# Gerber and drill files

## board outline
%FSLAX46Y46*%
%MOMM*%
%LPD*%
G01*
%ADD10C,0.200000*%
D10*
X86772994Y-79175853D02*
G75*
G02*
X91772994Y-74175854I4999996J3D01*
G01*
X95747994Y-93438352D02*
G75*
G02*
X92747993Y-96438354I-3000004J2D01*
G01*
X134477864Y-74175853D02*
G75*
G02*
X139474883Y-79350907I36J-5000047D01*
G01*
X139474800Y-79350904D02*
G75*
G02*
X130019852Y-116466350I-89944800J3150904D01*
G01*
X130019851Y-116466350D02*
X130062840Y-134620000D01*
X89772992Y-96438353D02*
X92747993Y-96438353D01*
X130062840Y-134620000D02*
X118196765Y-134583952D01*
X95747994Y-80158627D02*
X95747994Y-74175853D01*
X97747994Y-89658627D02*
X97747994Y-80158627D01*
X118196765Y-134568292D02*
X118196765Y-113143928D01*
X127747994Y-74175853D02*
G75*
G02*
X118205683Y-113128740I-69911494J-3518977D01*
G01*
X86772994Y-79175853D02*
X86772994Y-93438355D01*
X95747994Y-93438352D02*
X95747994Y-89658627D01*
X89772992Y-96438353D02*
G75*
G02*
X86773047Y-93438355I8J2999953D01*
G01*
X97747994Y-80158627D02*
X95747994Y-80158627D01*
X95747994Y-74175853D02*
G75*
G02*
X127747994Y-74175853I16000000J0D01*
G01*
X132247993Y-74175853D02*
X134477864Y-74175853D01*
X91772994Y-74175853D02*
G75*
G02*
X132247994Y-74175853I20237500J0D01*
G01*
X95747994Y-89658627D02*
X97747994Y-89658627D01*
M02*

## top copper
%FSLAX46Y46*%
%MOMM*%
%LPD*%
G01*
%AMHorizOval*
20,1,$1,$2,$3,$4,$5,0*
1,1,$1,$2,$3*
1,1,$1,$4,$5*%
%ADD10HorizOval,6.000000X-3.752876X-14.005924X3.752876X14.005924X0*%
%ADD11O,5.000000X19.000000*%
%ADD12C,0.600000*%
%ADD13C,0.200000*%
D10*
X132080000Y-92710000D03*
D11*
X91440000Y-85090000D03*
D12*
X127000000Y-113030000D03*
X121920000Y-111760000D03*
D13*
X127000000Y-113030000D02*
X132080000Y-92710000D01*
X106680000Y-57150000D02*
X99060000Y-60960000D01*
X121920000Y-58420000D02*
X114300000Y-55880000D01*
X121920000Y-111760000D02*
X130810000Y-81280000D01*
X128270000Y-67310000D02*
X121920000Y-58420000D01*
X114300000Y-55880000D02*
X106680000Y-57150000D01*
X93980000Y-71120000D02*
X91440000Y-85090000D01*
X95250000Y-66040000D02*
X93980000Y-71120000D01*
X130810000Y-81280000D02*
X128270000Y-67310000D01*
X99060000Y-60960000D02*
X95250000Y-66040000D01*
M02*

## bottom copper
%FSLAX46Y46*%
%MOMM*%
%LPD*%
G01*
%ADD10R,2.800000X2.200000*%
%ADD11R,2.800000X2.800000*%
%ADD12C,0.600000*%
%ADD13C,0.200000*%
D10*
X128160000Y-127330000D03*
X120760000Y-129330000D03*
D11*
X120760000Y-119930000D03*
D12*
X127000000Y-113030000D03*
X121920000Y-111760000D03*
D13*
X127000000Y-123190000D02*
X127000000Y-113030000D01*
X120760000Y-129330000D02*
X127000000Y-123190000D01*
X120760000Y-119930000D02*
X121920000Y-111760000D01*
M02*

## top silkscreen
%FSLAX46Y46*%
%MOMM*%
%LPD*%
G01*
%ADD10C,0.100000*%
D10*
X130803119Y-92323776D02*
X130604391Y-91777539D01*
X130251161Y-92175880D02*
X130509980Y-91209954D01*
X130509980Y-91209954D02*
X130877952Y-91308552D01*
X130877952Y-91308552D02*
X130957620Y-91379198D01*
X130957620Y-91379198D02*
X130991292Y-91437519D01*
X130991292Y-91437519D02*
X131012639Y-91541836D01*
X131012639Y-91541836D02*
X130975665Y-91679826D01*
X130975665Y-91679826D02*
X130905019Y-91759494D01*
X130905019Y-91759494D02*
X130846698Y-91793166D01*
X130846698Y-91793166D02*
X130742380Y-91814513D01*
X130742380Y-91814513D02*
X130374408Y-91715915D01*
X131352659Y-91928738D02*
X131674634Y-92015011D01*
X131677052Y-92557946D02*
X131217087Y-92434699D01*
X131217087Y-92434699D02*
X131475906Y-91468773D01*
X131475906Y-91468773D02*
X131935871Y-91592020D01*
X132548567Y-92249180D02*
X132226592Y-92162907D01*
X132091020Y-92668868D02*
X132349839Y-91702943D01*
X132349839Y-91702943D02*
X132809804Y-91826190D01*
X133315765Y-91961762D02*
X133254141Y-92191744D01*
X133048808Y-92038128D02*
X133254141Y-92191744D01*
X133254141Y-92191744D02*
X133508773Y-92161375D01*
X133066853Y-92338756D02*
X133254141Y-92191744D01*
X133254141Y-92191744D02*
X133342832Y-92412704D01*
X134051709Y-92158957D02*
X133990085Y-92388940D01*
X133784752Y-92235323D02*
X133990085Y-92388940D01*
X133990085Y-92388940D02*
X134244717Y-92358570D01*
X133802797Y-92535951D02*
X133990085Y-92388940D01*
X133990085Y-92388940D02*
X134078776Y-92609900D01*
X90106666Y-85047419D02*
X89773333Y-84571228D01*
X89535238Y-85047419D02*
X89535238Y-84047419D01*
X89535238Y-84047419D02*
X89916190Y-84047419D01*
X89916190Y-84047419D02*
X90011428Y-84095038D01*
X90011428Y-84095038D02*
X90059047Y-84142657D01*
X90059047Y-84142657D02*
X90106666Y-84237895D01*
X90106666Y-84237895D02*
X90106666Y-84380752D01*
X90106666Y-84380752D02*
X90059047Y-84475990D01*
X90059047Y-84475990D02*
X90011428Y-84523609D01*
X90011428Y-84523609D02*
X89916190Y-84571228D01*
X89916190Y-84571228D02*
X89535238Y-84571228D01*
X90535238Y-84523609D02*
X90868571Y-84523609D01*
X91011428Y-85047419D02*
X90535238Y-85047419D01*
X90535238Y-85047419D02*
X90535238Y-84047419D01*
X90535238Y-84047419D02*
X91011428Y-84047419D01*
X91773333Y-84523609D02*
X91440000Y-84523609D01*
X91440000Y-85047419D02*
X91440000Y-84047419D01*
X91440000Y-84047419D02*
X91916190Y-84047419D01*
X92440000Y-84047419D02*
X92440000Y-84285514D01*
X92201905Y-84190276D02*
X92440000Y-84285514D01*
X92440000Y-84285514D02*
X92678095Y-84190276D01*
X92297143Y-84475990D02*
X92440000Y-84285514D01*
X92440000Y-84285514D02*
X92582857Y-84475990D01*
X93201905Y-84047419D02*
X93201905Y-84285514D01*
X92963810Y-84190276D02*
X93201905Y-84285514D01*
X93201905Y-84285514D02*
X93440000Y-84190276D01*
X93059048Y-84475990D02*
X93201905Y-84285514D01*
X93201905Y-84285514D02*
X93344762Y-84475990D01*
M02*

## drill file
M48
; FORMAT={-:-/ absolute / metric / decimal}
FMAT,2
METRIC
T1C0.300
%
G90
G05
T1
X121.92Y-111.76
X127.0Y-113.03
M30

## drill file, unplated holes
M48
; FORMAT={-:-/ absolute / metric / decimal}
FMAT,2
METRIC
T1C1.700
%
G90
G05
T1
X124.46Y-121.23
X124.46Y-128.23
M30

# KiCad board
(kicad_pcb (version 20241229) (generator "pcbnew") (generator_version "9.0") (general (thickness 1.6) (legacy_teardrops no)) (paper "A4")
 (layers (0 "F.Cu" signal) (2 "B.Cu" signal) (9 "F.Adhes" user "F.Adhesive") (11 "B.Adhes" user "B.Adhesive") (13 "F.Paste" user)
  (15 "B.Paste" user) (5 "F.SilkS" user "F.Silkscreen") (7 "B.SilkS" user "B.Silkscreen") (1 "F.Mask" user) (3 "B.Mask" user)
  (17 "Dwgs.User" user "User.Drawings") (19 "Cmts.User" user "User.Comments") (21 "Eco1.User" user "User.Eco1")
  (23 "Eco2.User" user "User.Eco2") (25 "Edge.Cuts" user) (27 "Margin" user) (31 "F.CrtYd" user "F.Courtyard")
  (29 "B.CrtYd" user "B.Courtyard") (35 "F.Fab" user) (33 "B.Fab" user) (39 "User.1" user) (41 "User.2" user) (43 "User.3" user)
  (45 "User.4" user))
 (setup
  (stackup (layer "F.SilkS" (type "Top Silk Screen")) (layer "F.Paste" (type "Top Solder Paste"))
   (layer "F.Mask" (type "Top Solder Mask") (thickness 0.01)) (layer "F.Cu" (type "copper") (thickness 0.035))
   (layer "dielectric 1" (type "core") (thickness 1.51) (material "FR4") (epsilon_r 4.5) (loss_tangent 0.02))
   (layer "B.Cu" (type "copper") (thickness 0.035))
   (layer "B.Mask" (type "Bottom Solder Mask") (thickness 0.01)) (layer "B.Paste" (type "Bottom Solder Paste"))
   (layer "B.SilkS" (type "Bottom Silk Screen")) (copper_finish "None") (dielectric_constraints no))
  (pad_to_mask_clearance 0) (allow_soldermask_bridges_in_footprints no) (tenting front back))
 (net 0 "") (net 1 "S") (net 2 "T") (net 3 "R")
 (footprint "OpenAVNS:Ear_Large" (layer "F.Cu") (at 132.08 92.71 -15)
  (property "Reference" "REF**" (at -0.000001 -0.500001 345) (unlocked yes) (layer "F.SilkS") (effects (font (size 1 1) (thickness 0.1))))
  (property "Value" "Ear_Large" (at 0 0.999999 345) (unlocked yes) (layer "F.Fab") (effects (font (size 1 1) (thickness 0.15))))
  (pad "1" smd oval (at 0 0 345) (size 6 35) (layers "F.Cu" "F.Mask" "F.Paste") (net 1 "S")))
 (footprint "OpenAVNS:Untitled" (layer "F.Cu") (at 91.44 85.09)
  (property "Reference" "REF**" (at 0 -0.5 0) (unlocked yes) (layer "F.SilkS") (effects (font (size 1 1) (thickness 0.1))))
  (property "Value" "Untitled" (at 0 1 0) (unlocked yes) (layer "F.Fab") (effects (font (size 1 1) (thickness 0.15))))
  (pad "1" smd oval (at 0 0) (size 5 19) (layers "F.Cu" "F.Mask" "F.Paste") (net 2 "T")))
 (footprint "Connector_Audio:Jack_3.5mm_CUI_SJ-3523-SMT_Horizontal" (layer "B.Cu") (at 124.46 125.73)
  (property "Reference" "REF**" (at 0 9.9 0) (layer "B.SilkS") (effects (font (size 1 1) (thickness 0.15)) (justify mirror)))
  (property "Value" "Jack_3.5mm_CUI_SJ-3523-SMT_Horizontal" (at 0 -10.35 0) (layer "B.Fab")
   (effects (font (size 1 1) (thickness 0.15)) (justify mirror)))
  (pad "" np_thru_hole circle (at 0 -4.5) (size 1.7 1.7) (drill 1.7) (layers "*.Cu" "*.Mask"))
  (pad "" np_thru_hole circle (at 0 2.5) (size 1.7 1.7) (drill 1.7) (layers "*.Cu" "*.Mask"))
  (pad "R" smd rect (at 3.7 1.6) (size 2.8 2.2) (layers "B.Cu" "B.Mask" "B.Paste") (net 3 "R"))
  (pad "S" smd rect (at -3.7 3.6) (size 2.8 2.2) (layers "B.Cu" "B.Mask" "B.Paste") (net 1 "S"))
  (pad "T" smd rect (at -3.7 -5.8) (size 2.8 2.8) (layers "B.Cu" "B.Mask" "B.Paste") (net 2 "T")))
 (gr_arc (start 86.772994 79.175853) (mid 88.23746 75.640319) (end 91.772994 74.175853) (stroke (width 0.2) (type default))
  (layer "Edge.Cuts"))
 (gr_arc (start 95.747994 93.438352) (mid 94.869314 95.559673) (end 92.747993 96.438353) (stroke (width 0.2) (type default))
  (layer "Edge.Cuts"))
 (gr_arc (start 134.477864 74.175853) (mid 138.074756 75.702761) (end 139.4748 79.350904) (stroke (width 0.2) (type default))
  (layer "Edge.Cuts"))
 (gr_arc (start 139.4748 79.350904) (mid 136.744573 98.417414) (end 130.019852 116.46635) (stroke (width 0.2) (type default))
  (layer "Edge.Cuts"))
 (gr_line (start 130.019851 116.46635) (end 130.06284 134.62) (stroke (width 0.2) (type default)) (layer "Edge.Cuts"))
 (gr_line (start 89.772992 96.438353) (end 92.747993 96.438353) (stroke (width 0.2) (type default)) (layer "Edge.Cuts"))
 (gr_line (start 130.06284 134.62) (end 118.196765 134.583952) (stroke (width 0.2) (type default)) (layer "Edge.Cuts"))
 (gr_line (start 95.747994 80.158627) (end 95.747994 74.175853) (stroke (width 0.2) (type default)) (layer "Edge.Cuts"))
 (gr_line (start 97.747994 89.658627) (end 97.747994 80.158627) (stroke (width 0.2) (type default)) (layer "Edge.Cuts"))
 (gr_line (start 118.196765 134.568292) (end 118.196765 113.143928) (stroke (width 0.2) (type default)) (layer "Edge.Cuts"))
 (gr_arc (start 127.747994 74.175853) (mid 125.826173 94.3503) (end 118.205684 113.128741) (stroke (width 0.2) (type default))
  (layer "Edge.Cuts"))
 (gr_line (start 86.772994 79.175853) (end 86.772994 93.438355) (stroke (width 0.2) (type default)) (layer "Edge.Cuts"))
 (gr_line (start 95.747994 93.438352) (end 95.747994 89.658627) (stroke (width 0.2) (type default)) (layer "Edge.Cuts"))
 (gr_arc (start 89.772992 96.438353) (mid 87.651673 95.559674) (end 86.772994 93.438355) (stroke (width 0.2) (type default))
  (layer "Edge.Cuts"))
 (gr_line (start 97.747994 80.158627) (end 95.747994 80.158627) (stroke (width 0.2) (type default)) (layer "Edge.Cuts"))
 (gr_arc (start 95.747994 74.175853) (mid 111.747994 58.175853) (end 127.747994 74.175853) (stroke (width 0.2) (type default))
  (layer "Edge.Cuts"))
 (gr_line (start 132.247993 74.175853) (end 134.477864 74.175853) (stroke (width 0.2) (type default)) (layer "Edge.Cuts"))
 (gr_arc (start 91.772994 74.175853) (mid 112.010494 53.938353) (end 132.247993 74.175853) (stroke (width 0.2) (type default))
  (layer "Edge.Cuts"))
 (gr_line (start 95.747994 89.658627) (end 97.747994 89.658627) (stroke (width 0.2) (type default)) (layer "Edge.Cuts"))
 (segment (start 95.25 66.04) (end 93.98 71.12) (width 0.2) (layer "F.Cu") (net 2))
 (segment (start 106.68 57.15) (end 99.06 60.96) (width 0.2) (layer "F.Cu") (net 2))
 (segment (start 121.92 58.42) (end 114.3 55.88) (width 0.2) (layer "F.Cu") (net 2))
 (segment (start 128.27 67.31) (end 121.92 58.42) (width 0.2) (layer "F.Cu") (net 2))
 (segment (start 121.92 111.76) (end 130.81 81.28) (width 0.2) (layer "F.Cu") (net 2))
 (segment (start 130.81 81.28) (end 128.27 67.31) (width 0.2) (layer "F.Cu") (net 2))
 (segment (start 114.3 55.88) (end 106.68 57.15) (width 0.2) (layer "F.Cu") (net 2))
 (segment (start 99.06 60.96) (end 95.25 66.04) (width 0.2) (layer "F.Cu") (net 2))
 (segment (start 93.98 71.12) (end 91.44 85.09) (width 0.2) (layer "F.Cu") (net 2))
 (via (at 121.92 111.76) (size 0.6) (drill 0.3) (layers "F.Cu" "B.Cu") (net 2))
 (segment (start 120.76 119.93) (end 121.92 111.76) (width 0.2) (layer "B.Cu") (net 2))
 (segment (start 127 113.03) (end 132.08 92.71) (width 0.2) (layer "F.Cu") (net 1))
 (via (at 127 113.03) (size 0.6) (drill 0.3) (layers "F.Cu" "B.Cu") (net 1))
 (segment (start 127 123.19) (end 127 113.03) (width 0.2) (layer "B.Cu") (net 1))
 (segment (start 120.76 129.33) (end 127 123.19) (width 0.2) (layer "B.Cu") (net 1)))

